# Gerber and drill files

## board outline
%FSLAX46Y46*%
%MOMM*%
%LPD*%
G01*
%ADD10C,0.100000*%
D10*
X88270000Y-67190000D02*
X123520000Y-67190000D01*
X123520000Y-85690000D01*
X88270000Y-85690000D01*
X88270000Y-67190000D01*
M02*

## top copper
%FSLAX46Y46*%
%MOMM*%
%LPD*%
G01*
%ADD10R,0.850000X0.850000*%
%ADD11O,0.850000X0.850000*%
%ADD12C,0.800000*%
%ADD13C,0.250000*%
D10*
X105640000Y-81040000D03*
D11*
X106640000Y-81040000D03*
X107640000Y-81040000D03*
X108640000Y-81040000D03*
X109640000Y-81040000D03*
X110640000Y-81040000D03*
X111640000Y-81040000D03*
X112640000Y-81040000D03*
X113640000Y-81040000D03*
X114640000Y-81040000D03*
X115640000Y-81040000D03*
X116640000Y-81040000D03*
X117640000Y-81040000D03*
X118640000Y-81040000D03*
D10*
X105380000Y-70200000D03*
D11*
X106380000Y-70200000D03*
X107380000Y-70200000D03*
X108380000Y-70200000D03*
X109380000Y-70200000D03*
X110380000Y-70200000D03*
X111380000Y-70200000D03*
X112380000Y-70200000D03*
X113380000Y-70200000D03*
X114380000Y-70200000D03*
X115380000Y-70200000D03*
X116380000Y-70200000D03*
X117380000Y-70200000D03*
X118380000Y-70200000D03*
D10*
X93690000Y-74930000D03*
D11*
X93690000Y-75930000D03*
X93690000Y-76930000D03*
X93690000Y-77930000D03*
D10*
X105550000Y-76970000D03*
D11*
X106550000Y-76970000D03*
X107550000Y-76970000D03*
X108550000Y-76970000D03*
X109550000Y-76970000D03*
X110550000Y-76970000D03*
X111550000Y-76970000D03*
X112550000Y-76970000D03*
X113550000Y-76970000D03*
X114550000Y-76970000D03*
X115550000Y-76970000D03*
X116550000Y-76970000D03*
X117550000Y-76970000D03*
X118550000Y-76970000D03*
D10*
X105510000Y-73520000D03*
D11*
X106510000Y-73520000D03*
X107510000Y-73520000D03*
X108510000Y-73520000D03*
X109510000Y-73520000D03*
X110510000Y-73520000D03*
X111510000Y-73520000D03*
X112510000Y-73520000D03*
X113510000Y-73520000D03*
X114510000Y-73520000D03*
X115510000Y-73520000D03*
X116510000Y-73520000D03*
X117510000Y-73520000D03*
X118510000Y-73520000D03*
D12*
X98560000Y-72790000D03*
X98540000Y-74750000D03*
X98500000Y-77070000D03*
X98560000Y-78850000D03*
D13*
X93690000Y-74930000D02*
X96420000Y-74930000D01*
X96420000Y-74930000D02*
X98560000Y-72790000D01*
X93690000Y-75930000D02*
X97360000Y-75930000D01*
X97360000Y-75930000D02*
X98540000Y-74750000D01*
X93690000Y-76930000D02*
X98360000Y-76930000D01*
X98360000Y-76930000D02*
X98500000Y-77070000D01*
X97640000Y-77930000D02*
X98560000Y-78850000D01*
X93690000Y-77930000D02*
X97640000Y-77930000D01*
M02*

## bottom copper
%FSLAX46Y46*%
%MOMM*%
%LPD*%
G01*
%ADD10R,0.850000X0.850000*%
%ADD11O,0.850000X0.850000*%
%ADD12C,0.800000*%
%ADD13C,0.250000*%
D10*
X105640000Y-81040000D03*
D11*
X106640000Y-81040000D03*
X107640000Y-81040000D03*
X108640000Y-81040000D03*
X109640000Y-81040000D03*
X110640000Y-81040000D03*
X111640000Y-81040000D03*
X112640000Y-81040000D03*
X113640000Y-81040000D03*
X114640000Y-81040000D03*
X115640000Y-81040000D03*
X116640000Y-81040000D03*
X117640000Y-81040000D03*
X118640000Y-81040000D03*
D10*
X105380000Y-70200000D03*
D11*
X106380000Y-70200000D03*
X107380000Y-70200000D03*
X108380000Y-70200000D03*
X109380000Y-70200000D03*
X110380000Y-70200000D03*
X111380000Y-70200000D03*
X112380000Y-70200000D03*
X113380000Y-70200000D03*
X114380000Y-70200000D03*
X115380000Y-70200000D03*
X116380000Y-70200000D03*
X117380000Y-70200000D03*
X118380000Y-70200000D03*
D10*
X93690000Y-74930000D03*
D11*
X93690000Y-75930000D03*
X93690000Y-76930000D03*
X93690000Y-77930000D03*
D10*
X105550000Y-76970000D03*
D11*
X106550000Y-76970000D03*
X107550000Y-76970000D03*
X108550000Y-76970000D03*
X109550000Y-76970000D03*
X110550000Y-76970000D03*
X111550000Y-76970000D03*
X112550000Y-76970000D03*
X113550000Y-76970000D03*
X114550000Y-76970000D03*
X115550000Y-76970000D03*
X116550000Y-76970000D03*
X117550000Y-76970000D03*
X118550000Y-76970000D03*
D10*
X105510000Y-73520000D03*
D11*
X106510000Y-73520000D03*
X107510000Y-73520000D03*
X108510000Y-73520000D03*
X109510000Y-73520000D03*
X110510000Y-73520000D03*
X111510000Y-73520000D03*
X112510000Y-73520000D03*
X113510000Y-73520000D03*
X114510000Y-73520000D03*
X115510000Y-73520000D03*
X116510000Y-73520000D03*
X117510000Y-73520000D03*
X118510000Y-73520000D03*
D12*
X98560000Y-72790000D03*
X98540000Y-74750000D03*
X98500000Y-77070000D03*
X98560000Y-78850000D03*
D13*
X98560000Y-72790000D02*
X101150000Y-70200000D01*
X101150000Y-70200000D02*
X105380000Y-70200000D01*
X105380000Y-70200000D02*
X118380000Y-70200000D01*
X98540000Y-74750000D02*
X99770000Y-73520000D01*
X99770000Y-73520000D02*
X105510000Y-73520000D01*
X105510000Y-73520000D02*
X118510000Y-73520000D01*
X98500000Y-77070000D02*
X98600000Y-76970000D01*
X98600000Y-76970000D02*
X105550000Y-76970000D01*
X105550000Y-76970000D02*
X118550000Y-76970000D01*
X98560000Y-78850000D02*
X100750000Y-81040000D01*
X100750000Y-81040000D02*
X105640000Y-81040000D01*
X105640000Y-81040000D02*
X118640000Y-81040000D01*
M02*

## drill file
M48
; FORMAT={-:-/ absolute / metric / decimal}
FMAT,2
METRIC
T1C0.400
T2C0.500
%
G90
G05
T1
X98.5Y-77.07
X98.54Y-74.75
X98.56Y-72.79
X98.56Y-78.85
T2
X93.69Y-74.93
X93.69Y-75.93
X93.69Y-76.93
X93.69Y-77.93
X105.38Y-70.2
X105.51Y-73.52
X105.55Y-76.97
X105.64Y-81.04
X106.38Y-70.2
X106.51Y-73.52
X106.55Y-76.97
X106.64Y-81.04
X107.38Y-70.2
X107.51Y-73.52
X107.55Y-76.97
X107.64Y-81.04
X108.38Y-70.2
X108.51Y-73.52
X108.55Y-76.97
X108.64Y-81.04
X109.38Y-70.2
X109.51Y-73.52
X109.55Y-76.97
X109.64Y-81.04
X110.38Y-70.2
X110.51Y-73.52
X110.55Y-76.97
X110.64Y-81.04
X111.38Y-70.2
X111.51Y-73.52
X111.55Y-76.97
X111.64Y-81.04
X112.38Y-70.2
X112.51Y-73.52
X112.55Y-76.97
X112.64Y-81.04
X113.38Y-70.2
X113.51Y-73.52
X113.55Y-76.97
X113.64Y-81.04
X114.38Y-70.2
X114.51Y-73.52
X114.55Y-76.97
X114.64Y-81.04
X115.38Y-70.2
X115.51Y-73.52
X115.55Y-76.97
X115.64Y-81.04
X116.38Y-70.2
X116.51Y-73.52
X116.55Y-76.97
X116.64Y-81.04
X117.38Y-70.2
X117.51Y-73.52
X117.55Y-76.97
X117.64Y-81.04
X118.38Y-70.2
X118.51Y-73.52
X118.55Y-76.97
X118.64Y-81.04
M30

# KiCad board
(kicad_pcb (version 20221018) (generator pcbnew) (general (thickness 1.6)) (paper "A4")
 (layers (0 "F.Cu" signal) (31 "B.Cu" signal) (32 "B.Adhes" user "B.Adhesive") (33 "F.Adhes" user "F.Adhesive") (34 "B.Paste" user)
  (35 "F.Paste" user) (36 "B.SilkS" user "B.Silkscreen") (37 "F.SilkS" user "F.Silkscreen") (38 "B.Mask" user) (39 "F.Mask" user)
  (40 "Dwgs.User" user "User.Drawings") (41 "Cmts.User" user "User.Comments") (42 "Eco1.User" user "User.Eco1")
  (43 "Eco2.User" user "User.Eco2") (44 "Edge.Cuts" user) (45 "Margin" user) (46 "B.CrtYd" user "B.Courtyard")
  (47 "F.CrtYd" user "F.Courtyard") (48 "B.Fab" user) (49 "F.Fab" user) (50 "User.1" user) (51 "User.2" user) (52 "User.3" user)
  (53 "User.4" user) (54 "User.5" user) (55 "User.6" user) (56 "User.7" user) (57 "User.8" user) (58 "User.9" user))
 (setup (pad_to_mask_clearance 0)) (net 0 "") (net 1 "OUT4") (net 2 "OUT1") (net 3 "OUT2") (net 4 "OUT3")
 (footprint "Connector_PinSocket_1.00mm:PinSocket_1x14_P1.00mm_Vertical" (layer "F.Cu") (at 105.64 81.04 90)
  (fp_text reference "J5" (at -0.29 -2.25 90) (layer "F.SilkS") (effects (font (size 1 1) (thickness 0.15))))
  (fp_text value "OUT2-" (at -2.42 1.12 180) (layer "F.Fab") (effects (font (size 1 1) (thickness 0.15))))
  (pad "1" thru_hole rect (at 0 0 90) (size 0.85 0.85) (drill 0.5) (layers "*.Cu" "*.Mask") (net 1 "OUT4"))
  (pad "2" thru_hole oval (at 0 1 90) (size 0.85 0.85) (drill 0.5) (layers "*.Cu" "*.Mask") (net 1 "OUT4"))
  (pad "3" thru_hole oval (at 0 2 90) (size 0.85 0.85) (drill 0.5) (layers "*.Cu" "*.Mask") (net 1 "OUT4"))
  (pad "4" thru_hole oval (at 0 3 90) (size 0.85 0.85) (drill 0.5) (layers "*.Cu" "*.Mask") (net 1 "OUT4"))
  (pad "5" thru_hole oval (at 0 4 90) (size 0.85 0.85) (drill 0.5) (layers "*.Cu" "*.Mask") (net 1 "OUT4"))
  (pad "6" thru_hole oval (at 0 5 90) (size 0.85 0.85) (drill 0.5) (layers "*.Cu" "*.Mask") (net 1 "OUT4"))
  (pad "7" thru_hole oval (at 0 6 90) (size 0.85 0.85) (drill 0.5) (layers "*.Cu" "*.Mask") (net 1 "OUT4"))
  (pad "8" thru_hole oval (at 0 7 90) (size 0.85 0.85) (drill 0.5) (layers "*.Cu" "*.Mask") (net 1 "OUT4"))
  (pad "9" thru_hole oval (at 0 8 90) (size 0.85 0.85) (drill 0.5) (layers "*.Cu" "*.Mask") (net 1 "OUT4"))
  (pad "10" thru_hole oval (at 0 9 90) (size 0.85 0.85) (drill 0.5) (layers "*.Cu" "*.Mask") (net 1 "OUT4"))
  (pad "11" thru_hole oval (at 0 10 90) (size 0.85 0.85) (drill 0.5) (layers "*.Cu" "*.Mask") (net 1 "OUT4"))
  (pad "12" thru_hole oval (at 0 11 90) (size 0.85 0.85) (drill 0.5) (layers "*.Cu" "*.Mask") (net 1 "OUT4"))
  (pad "13" thru_hole oval (at 0 12 90) (size 0.85 0.85) (drill 0.5) (layers "*.Cu" "*.Mask") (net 1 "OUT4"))
  (pad "14" thru_hole oval (at 0 13 90) (size 0.85 0.85) (drill 0.5) (layers "*.Cu" "*.Mask") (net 1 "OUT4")))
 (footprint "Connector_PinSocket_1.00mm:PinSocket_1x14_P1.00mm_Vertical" (layer "F.Cu") (at 105.38 70.2 90)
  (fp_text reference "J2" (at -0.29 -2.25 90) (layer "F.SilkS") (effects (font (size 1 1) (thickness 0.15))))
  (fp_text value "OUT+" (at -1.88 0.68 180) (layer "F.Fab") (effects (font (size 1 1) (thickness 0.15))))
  (pad "1" thru_hole rect (at 0 0 90) (size 0.85 0.85) (drill 0.5) (layers "*.Cu" "*.Mask") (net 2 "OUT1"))
  (pad "2" thru_hole oval (at 0 1 90) (size 0.85 0.85) (drill 0.5) (layers "*.Cu" "*.Mask") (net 2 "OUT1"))
  (pad "3" thru_hole oval (at 0 2 90) (size 0.85 0.85) (drill 0.5) (layers "*.Cu" "*.Mask") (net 2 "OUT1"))
  (pad "4" thru_hole oval (at 0 3 90) (size 0.85 0.85) (drill 0.5) (layers "*.Cu" "*.Mask") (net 2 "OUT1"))
  (pad "5" thru_hole oval (at 0 4 90) (size 0.85 0.85) (drill 0.5) (layers "*.Cu" "*.Mask") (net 2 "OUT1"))
  (pad "6" thru_hole oval (at 0 5 90) (size 0.85 0.85) (drill 0.5) (layers "*.Cu" "*.Mask") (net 2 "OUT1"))
  (pad "7" thru_hole oval (at 0 6 90) (size 0.85 0.85) (drill 0.5) (layers "*.Cu" "*.Mask") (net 2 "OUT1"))
  (pad "8" thru_hole oval (at 0 7 90) (size 0.85 0.85) (drill 0.5) (layers "*.Cu" "*.Mask") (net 2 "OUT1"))
  (pad "9" thru_hole oval (at 0 8 90) (size 0.85 0.85) (drill 0.5) (layers "*.Cu" "*.Mask") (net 2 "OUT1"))
  (pad "10" thru_hole oval (at 0 9 90) (size 0.85 0.85) (drill 0.5) (layers "*.Cu" "*.Mask") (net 2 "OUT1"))
  (pad "11" thru_hole oval (at 0 10 90) (size 0.85 0.85) (drill 0.5) (layers "*.Cu" "*.Mask") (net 2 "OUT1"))
  (pad "12" thru_hole oval (at 0 11 90) (size 0.85 0.85) (drill 0.5) (layers "*.Cu" "*.Mask") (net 2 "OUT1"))
  (pad "13" thru_hole oval (at 0 12 90) (size 0.85 0.85) (drill 0.5) (layers "*.Cu" "*.Mask") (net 2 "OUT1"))
  (pad "14" thru_hole oval (at 0 13 90) (size 0.85 0.85) (drill 0.5) (layers "*.Cu" "*.Mask") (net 2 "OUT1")))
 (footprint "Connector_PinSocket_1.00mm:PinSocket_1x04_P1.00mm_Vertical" (layer "F.Cu") (at 93.69 74.93)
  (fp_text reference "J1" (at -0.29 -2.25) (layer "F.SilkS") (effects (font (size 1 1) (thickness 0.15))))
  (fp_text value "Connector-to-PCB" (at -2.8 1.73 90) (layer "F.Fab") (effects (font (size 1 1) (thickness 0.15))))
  (pad "1" thru_hole rect (at 0 0) (size 0.85 0.85) (drill 0.5) (layers "*.Cu" "*.Mask") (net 2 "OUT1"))
  (pad "2" thru_hole oval (at 0 1) (size 0.85 0.85) (drill 0.5) (layers "*.Cu" "*.Mask") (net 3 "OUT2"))
  (pad "3" thru_hole oval (at 0 2) (size 0.85 0.85) (drill 0.5) (layers "*.Cu" "*.Mask") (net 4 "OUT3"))
  (pad "4" thru_hole oval (at 0 3) (size 0.85 0.85) (drill 0.5) (layers "*.Cu" "*.Mask") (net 1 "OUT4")))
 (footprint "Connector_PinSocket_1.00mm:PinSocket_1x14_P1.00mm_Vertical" (layer "F.Cu") (at 105.55 76.97 90)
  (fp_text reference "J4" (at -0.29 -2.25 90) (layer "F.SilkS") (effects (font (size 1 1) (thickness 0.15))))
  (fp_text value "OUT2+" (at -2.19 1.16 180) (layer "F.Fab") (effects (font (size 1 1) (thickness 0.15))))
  (pad "1" thru_hole rect (at 0 0 90) (size 0.85 0.85) (drill 0.5) (layers "*.Cu" "*.Mask") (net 4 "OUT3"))
  (pad "2" thru_hole oval (at 0 1 90) (size 0.85 0.85) (drill 0.5) (layers "*.Cu" "*.Mask") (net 4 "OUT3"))
  (pad "3" thru_hole oval (at 0 2 90) (size 0.85 0.85) (drill 0.5) (layers "*.Cu" "*.Mask") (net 4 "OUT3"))
  (pad "4" thru_hole oval (at 0 3 90) (size 0.85 0.85) (drill 0.5) (layers "*.Cu" "*.Mask") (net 4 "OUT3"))
  (pad "5" thru_hole oval (at 0 4 90) (size 0.85 0.85) (drill 0.5) (layers "*.Cu" "*.Mask") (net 4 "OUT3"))
  (pad "6" thru_hole oval (at 0 5 90) (size 0.85 0.85) (drill 0.5) (layers "*.Cu" "*.Mask") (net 4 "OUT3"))
  (pad "7" thru_hole oval (at 0 6 90) (size 0.85 0.85) (drill 0.5) (layers "*.Cu" "*.Mask") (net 4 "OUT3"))
  (pad "8" thru_hole oval (at 0 7 90) (size 0.85 0.85) (drill 0.5) (layers "*.Cu" "*.Mask") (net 4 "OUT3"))
  (pad "9" thru_hole oval (at 0 8 90) (size 0.85 0.85) (drill 0.5) (layers "*.Cu" "*.Mask") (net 4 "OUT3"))
  (pad "10" thru_hole oval (at 0 9 90) (size 0.85 0.85) (drill 0.5) (layers "*.Cu" "*.Mask") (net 4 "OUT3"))
  (pad "11" thru_hole oval (at 0 10 90) (size 0.85 0.85) (drill 0.5) (layers "*.Cu" "*.Mask") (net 4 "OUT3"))
  (pad "12" thru_hole oval (at 0 11 90) (size 0.85 0.85) (drill 0.5) (layers "*.Cu" "*.Mask") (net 4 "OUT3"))
  (pad "13" thru_hole oval (at 0 12 90) (size 0.85 0.85) (drill 0.5) (layers "*.Cu" "*.Mask") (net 4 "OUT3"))
  (pad "14" thru_hole oval (at 0 13 90) (size 0.85 0.85) (drill 0.5) (layers "*.Cu" "*.Mask") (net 4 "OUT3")))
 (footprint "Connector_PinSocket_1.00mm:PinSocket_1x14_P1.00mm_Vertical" (layer "F.Cu") (at 105.51 73.52 90)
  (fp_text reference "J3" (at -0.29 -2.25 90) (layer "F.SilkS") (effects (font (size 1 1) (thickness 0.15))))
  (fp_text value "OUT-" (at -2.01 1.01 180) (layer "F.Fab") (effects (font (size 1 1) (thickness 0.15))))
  (pad "1" thru_hole rect (at 0 0 90) (size 0.85 0.85) (drill 0.5) (layers "*.Cu" "*.Mask") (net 3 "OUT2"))
  (pad "2" thru_hole oval (at 0 1 90) (size 0.85 0.85) (drill 0.5) (layers "*.Cu" "*.Mask") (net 3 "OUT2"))
  (pad "3" thru_hole oval (at 0 2 90) (size 0.85 0.85) (drill 0.5) (layers "*.Cu" "*.Mask") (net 3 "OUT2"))
  (pad "4" thru_hole oval (at 0 3 90) (size 0.85 0.85) (drill 0.5) (layers "*.Cu" "*.Mask") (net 3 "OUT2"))
  (pad "5" thru_hole oval (at 0 4 90) (size 0.85 0.85) (drill 0.5) (layers "*.Cu" "*.Mask") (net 3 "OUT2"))
  (pad "6" thru_hole oval (at 0 5 90) (size 0.85 0.85) (drill 0.5) (layers "*.Cu" "*.Mask") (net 3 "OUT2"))
  (pad "7" thru_hole oval (at 0 6 90) (size 0.85 0.85) (drill 0.5) (layers "*.Cu" "*.Mask") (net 3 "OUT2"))
  (pad "8" thru_hole oval (at 0 7 90) (size 0.85 0.85) (drill 0.5) (layers "*.Cu" "*.Mask") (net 3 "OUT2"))
  (pad "9" thru_hole oval (at 0 8 90) (size 0.85 0.85) (drill 0.5) (layers "*.Cu" "*.Mask") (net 3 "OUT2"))
  (pad "10" thru_hole oval (at 0 9 90) (size 0.85 0.85) (drill 0.5) (layers "*.Cu" "*.Mask") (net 3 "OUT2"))
  (pad "11" thru_hole oval (at 0 10 90) (size 0.85 0.85) (drill 0.5) (layers "*.Cu" "*.Mask") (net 3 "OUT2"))
  (pad "12" thru_hole oval (at 0 11 90) (size 0.85 0.85) (drill 0.5) (layers "*.Cu" "*.Mask") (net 3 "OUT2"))
  (pad "13" thru_hole oval (at 0 12 90) (size 0.85 0.85) (drill 0.5) (layers "*.Cu" "*.Mask") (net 3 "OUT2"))
  (pad "14" thru_hole oval (at 0 13 90) (size 0.85 0.85) (drill 0.5) (layers "*.Cu" "*.Mask") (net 3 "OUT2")))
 (gr_rect (start 88.27 67.19) (end 123.52 85.69) (stroke (width 0.1) (type default)) (fill none) (layer "Edge.Cuts"))
 (segment (start 93.69 74.93) (end 96.42 74.93) (width 0.25) (layer "F.Cu") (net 2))
 (segment (start 96.42 74.93) (end 98.56 72.79) (width 0.25) (layer "F.Cu") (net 2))
 (via (at 98.56 72.79) (size 0.8) (drill 0.4) (layers "F.Cu" "B.Cu") (free) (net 2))
 (segment (start 98.56 72.79) (end 101.15 70.2) (width 0.25) (layer "B.Cu") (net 2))
 (segment (start 101.15 70.2) (end 105.38 70.2) (width 0.25) (layer "B.Cu") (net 2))
 (segment (start 105.38 70.2) (end 118.38 70.2) (width 0.25) (layer "B.Cu") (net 2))
 (segment (start 93.69 75.93) (end 97.36 75.93) (width 0.25) (layer "F.Cu") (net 3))
 (segment (start 97.36 75.93) (end 98.54 74.75) (width 0.25) (layer "F.Cu") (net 3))
 (via (at 98.54 74.75) (size 0.8) (drill 0.4) (layers "F.Cu" "B.Cu") (free) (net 3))
 (segment (start 98.54 74.75) (end 99.77 73.52) (width 0.25) (layer "B.Cu") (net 3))
 (segment (start 99.77 73.52) (end 105.51 73.52) (width 0.25) (layer "B.Cu") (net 3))
 (segment (start 105.51 73.52) (end 118.51 73.52) (width 0.25) (layer "B.Cu") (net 3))
 (segment (start 93.69 76.93) (end 98.36 76.93) (width 0.25) (layer "F.Cu") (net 4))
 (segment (start 98.36 76.93) (end 98.5 77.07) (width 0.25) (layer "F.Cu") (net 4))
 (via (at 98.5 77.07) (size 0.8) (drill 0.4) (layers "F.Cu" "B.Cu") (free) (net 4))
 (segment (start 98.5 77.07) (end 98.6 76.97) (width 0.25) (layer "B.Cu") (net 4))
 (segment (start 98.6 76.97) (end 105.55 76.97) (width 0.25) (layer "B.Cu") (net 4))
 (segment (start 105.55 76.97) (end 118.55 76.97) (width 0.25) (layer "B.Cu") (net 4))
 (segment (start 97.64 77.93) (end 98.56 78.85) (width 0.25) (layer "F.Cu") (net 1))
 (segment (start 93.69 77.93) (end 97.64 77.93) (width 0.25) (layer "F.Cu") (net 1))
 (via (at 98.56 78.85) (size 0.8) (drill 0.4) (layers "F.Cu" "B.Cu") (free) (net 1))
 (segment (start 98.56 78.85) (end 100.75 81.04) (width 0.25) (layer "B.Cu") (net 1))
 (segment (start 100.75 81.04) (end 105.64 81.04) (width 0.25) (layer "B.Cu") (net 1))
 (segment (start 105.64 81.04) (end 118.64 81.04) (width 0.25) (layer "B.Cu") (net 1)))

